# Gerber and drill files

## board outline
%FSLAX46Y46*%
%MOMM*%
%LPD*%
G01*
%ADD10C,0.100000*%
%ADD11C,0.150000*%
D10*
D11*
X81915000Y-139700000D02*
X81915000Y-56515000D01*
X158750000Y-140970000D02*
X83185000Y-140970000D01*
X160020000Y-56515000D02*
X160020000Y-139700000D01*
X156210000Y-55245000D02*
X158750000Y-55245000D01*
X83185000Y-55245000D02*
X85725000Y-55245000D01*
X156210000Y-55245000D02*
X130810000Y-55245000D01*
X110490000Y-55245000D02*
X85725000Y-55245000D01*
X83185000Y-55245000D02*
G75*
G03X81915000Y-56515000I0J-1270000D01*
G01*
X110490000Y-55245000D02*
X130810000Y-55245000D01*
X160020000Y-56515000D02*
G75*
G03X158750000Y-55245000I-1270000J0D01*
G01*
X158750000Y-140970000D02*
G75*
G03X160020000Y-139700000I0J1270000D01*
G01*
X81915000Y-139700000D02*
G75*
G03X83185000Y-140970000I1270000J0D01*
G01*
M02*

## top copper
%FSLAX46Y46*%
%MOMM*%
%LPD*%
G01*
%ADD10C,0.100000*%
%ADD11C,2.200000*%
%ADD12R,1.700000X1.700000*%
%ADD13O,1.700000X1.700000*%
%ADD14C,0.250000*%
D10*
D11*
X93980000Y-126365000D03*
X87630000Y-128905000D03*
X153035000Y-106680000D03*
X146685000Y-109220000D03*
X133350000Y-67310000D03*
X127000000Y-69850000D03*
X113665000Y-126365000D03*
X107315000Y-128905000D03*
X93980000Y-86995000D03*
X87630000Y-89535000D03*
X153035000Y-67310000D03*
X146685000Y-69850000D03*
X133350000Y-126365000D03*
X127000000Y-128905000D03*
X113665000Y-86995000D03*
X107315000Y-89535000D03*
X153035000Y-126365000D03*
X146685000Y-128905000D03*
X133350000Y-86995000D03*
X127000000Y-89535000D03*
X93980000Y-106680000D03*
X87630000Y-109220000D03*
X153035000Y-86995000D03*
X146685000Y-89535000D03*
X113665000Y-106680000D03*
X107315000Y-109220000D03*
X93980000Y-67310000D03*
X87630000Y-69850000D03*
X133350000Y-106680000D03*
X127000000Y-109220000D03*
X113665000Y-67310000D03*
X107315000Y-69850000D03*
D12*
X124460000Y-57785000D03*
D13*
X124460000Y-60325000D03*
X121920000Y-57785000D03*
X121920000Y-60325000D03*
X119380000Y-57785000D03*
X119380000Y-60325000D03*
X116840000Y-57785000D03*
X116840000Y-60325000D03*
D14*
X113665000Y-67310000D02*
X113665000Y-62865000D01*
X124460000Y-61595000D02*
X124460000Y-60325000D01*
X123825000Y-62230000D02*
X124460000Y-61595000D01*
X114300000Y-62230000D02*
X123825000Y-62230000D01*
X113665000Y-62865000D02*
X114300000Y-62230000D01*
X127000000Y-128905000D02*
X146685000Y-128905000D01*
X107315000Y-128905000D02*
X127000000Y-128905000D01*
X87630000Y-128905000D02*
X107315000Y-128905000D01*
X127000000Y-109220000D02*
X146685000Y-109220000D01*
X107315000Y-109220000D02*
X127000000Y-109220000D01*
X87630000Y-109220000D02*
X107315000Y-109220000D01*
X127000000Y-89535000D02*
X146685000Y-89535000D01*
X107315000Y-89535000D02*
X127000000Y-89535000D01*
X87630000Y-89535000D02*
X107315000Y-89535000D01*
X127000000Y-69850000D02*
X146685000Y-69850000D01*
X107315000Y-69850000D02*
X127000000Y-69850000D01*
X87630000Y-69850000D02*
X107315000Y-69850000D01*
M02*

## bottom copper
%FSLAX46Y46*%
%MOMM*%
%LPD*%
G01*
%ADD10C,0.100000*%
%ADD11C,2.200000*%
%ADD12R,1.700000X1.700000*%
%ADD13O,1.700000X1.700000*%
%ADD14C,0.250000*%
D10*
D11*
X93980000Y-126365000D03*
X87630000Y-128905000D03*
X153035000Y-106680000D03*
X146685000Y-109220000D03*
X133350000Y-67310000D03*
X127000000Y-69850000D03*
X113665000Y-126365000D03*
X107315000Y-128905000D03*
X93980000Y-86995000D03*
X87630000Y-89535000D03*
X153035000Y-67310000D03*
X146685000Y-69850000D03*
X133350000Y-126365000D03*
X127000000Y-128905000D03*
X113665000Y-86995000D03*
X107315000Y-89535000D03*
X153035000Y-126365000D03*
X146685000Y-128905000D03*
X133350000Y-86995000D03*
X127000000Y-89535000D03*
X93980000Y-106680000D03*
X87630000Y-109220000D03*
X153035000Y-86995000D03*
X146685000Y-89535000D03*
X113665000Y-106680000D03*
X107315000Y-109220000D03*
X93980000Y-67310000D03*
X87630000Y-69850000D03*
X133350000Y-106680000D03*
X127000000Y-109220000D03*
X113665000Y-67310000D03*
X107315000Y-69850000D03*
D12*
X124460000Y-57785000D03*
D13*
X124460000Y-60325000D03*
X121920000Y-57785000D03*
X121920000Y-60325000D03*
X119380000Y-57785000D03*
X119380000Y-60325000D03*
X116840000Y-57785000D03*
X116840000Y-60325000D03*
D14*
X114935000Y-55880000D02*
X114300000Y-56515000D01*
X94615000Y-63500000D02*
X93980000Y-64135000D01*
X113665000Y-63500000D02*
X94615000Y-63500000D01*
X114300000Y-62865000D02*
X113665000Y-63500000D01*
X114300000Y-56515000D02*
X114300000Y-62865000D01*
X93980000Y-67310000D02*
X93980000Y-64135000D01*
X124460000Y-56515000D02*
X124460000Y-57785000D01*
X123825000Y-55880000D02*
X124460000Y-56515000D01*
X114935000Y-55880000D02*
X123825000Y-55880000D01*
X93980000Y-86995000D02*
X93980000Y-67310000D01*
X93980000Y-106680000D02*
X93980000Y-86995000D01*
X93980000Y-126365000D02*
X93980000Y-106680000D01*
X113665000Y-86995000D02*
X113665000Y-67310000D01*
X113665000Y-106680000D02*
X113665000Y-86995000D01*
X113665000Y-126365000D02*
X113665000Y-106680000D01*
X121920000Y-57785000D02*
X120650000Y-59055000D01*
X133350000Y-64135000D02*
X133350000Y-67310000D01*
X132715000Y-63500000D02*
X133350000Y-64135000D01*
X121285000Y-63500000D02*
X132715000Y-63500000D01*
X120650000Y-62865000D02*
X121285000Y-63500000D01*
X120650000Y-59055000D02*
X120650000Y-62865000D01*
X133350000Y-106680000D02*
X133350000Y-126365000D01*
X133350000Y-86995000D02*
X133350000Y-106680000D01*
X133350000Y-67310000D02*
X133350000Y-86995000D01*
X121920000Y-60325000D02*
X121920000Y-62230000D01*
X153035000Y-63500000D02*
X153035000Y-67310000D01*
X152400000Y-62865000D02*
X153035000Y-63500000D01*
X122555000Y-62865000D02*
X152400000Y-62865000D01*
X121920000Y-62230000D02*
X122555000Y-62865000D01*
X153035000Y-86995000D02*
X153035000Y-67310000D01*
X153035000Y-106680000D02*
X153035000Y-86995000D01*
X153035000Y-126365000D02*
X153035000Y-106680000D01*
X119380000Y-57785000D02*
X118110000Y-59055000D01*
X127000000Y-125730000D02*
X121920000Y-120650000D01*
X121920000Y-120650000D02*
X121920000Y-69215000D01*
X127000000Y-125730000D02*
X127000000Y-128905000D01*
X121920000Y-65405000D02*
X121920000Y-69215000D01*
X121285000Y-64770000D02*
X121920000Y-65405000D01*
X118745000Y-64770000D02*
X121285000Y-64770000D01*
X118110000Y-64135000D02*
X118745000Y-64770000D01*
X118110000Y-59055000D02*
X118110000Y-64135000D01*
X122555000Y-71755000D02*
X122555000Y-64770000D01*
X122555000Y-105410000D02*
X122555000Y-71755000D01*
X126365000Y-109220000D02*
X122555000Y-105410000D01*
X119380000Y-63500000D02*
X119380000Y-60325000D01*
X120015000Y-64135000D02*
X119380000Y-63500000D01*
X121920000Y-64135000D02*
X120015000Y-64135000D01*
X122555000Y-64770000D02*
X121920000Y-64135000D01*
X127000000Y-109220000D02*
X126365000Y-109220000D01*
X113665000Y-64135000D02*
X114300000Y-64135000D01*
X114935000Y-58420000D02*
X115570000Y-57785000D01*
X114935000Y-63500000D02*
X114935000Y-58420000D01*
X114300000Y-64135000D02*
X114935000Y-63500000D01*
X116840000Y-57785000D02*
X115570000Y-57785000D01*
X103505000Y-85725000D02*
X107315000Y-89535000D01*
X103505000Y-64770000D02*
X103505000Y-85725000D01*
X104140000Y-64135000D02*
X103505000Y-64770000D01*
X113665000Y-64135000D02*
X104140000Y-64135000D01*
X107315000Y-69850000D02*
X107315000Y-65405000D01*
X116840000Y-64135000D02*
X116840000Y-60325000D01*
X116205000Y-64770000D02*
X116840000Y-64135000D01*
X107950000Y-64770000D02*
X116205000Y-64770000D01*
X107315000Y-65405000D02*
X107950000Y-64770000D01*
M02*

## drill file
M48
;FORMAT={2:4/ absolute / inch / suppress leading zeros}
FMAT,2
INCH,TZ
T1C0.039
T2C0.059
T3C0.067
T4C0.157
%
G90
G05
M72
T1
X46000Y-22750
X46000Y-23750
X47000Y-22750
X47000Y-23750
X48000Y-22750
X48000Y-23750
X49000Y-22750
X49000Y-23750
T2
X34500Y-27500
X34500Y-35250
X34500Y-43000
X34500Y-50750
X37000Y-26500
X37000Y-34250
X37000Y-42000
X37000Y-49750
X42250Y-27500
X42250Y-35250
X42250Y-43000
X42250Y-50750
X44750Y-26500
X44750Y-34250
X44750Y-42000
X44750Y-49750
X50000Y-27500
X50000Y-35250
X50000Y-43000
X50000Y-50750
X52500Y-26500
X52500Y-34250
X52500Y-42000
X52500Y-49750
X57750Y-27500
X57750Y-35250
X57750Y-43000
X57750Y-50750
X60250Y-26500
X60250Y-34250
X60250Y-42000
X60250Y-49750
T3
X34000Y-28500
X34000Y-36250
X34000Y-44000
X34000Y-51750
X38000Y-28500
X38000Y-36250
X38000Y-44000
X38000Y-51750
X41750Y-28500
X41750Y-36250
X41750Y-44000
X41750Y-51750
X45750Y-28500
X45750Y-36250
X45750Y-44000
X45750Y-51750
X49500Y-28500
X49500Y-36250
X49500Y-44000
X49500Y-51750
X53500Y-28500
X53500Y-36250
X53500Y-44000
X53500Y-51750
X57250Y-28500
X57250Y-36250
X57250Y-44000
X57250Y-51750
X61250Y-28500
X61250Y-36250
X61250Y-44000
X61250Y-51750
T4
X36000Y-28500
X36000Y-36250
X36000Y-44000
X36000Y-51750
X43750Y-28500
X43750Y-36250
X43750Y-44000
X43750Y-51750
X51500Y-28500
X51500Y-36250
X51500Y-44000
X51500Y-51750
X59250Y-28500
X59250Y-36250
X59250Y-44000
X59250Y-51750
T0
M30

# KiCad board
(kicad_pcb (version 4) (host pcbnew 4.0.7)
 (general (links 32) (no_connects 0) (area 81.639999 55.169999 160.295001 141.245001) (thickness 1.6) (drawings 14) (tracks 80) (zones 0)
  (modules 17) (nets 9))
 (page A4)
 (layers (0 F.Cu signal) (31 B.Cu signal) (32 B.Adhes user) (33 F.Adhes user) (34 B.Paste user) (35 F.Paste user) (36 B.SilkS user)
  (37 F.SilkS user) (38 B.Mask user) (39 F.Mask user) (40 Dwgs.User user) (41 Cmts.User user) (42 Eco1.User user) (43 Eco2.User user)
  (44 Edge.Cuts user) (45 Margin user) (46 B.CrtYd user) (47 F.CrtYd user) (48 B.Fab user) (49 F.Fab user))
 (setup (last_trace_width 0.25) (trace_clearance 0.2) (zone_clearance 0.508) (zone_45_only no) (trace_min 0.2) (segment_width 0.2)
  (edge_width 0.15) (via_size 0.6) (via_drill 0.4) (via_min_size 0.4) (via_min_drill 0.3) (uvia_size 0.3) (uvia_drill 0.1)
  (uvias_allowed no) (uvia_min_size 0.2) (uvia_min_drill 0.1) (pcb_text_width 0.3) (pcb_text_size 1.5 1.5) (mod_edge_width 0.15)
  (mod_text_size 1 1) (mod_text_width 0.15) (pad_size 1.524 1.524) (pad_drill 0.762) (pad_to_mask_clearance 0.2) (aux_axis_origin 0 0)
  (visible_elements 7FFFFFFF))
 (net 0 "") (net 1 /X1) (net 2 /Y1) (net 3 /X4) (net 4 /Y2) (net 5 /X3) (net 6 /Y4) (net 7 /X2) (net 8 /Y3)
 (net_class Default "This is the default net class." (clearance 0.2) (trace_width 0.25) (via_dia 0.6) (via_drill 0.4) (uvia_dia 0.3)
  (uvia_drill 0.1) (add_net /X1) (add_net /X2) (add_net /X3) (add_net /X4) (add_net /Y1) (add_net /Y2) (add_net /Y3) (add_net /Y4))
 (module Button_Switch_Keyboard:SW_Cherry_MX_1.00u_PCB (layer F.Cu) (at 93.98 126.365)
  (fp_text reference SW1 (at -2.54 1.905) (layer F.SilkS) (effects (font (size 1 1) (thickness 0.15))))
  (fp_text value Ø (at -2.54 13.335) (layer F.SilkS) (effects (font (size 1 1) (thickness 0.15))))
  (pad 1 thru_hole circle (at 0 0) (size 2.2 2.2) (drill 1.5) (layers *.Cu *.Mask) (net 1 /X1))
  (pad 2 thru_hole circle (at -6.35 2.54) (size 2.2 2.2) (drill 1.5) (layers *.Cu *.Mask) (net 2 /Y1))
  (pad "" np_thru_hole circle (at -2.54 5.08) (size 4 4) (drill 4) (layers *.Cu *.Mask))
  (pad "" np_thru_hole circle (at -7.62 5.08) (size 1.7 1.7) (drill 1.7) (layers *.Cu *.Mask))
  (pad "" np_thru_hole circle (at 2.54 5.08) (size 1.7 1.7) (drill 1.7) (layers *.Cu *.Mask)))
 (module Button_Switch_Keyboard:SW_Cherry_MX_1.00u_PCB (layer F.Cu) (at 153.035 106.68)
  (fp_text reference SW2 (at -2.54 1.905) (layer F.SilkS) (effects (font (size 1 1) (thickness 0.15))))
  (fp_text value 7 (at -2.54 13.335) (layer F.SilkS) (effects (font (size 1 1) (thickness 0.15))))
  (pad 1 thru_hole circle (at 0 0) (size 2.2 2.2) (drill 1.5) (layers *.Cu *.Mask) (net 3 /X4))
  (pad 2 thru_hole circle (at -6.35 2.54) (size 2.2 2.2) (drill 1.5) (layers *.Cu *.Mask) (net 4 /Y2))
  (pad "" np_thru_hole circle (at -2.54 5.08) (size 4 4) (drill 4) (layers *.Cu *.Mask))
  (pad "" np_thru_hole circle (at -7.62 5.08) (size 1.7 1.7) (drill 1.7) (layers *.Cu *.Mask))
  (pad "" np_thru_hole circle (at 2.54 5.08) (size 1.7 1.7) (drill 1.7) (layers *.Cu *.Mask)))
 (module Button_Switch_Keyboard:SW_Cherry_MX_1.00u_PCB (layer F.Cu) (at 133.35 67.31)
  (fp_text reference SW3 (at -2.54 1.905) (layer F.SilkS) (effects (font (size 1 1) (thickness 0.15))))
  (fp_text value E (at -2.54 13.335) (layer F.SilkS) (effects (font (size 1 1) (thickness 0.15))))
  (pad 1 thru_hole circle (at 0 0) (size 2.2 2.2) (drill 1.5) (layers *.Cu *.Mask) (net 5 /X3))
  (pad 2 thru_hole circle (at -6.35 2.54) (size 2.2 2.2) (drill 1.5) (layers *.Cu *.Mask) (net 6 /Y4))
  (pad "" np_thru_hole circle (at -2.54 5.08) (size 4 4) (drill 4) (layers *.Cu *.Mask))
  (pad "" np_thru_hole circle (at -7.62 5.08) (size 1.7 1.7) (drill 1.7) (layers *.Cu *.Mask))
  (pad "" np_thru_hole circle (at 2.54 5.08) (size 1.7 1.7) (drill 1.7) (layers *.Cu *.Mask)))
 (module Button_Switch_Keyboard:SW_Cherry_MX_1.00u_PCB (layer F.Cu) (at 113.665 126.365)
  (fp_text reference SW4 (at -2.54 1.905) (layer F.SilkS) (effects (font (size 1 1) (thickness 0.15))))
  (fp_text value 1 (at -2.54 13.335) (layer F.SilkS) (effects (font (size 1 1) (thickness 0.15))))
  (pad 1 thru_hole circle (at 0 0) (size 2.2 2.2) (drill 1.5) (layers *.Cu *.Mask) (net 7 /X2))
  (pad 2 thru_hole circle (at -6.35 2.54) (size 2.2 2.2) (drill 1.5) (layers *.Cu *.Mask) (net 2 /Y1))
  (pad "" np_thru_hole circle (at -2.54 5.08) (size 4 4) (drill 4) (layers *.Cu *.Mask))
  (pad "" np_thru_hole circle (at -7.62 5.08) (size 1.7 1.7) (drill 1.7) (layers *.Cu *.Mask))
  (pad "" np_thru_hole circle (at 2.54 5.08) (size 1.7 1.7) (drill 1.7) (layers *.Cu *.Mask)))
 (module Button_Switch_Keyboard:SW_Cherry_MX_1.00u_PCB (layer F.Cu) (at 93.98 86.995)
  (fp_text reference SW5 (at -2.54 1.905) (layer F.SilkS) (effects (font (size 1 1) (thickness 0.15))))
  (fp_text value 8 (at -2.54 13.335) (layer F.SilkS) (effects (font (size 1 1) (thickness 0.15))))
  (pad 1 thru_hole circle (at 0 0) (size 2.2 2.2) (drill 1.5) (layers *.Cu *.Mask) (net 1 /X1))
  (pad 2 thru_hole circle (at -6.35 2.54) (size 2.2 2.2) (drill 1.5) (layers *.Cu *.Mask) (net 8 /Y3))
  (pad "" np_thru_hole circle (at -2.54 5.08) (size 4 4) (drill 4) (layers *.Cu *.Mask))
  (pad "" np_thru_hole circle (at -7.62 5.08) (size 1.7 1.7) (drill 1.7) (layers *.Cu *.Mask))
  (pad "" np_thru_hole circle (at 2.54 5.08) (size 1.7 1.7) (drill 1.7) (layers *.Cu *.Mask)))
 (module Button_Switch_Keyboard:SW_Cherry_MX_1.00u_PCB (layer F.Cu) (at 153.035 67.31)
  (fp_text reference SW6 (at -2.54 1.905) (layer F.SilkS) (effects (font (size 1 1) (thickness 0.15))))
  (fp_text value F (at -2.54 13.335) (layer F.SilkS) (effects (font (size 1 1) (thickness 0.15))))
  (pad 1 thru_hole circle (at 0 0) (size 2.2 2.2) (drill 1.5) (layers *.Cu *.Mask) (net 3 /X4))
  (pad 2 thru_hole circle (at -6.35 2.54) (size 2.2 2.2) (drill 1.5) (layers *.Cu *.Mask) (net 6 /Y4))
  (pad "" np_thru_hole circle (at -2.54 5.08) (size 4 4) (drill 4) (layers *.Cu *.Mask))
  (pad "" np_thru_hole circle (at -7.62 5.08) (size 1.7 1.7) (drill 1.7) (layers *.Cu *.Mask))
  (pad "" np_thru_hole circle (at 2.54 5.08) (size 1.7 1.7) (drill 1.7) (layers *.Cu *.Mask)))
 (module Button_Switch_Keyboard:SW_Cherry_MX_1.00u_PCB (layer F.Cu) (at 133.35 126.365)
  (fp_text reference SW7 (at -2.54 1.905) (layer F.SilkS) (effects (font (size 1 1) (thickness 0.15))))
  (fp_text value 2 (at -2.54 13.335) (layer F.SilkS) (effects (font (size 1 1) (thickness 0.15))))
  (pad 1 thru_hole circle (at 0 0) (size 2.2 2.2) (drill 1.5) (layers *.Cu *.Mask) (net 5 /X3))
  (pad 2 thru_hole circle (at -6.35 2.54) (size 2.2 2.2) (drill 1.5) (layers *.Cu *.Mask) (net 2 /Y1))
  (pad "" np_thru_hole circle (at -2.54 5.08) (size 4 4) (drill 4) (layers *.Cu *.Mask))
  (pad "" np_thru_hole circle (at -7.62 5.08) (size 1.7 1.7) (drill 1.7) (layers *.Cu *.Mask))
  (pad "" np_thru_hole circle (at 2.54 5.08) (size 1.7 1.7) (drill 1.7) (layers *.Cu *.Mask)))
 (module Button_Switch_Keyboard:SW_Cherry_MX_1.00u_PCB (layer F.Cu) (at 113.665 86.995)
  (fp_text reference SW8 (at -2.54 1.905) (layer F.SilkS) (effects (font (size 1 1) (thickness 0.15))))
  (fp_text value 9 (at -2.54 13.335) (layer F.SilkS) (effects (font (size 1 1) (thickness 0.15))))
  (pad 1 thru_hole circle (at 0 0) (size 2.2 2.2) (drill 1.5) (layers *.Cu *.Mask) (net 7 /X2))
  (pad 2 thru_hole circle (at -6.35 2.54) (size 2.2 2.2) (drill 1.5) (layers *.Cu *.Mask) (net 8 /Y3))
  (pad "" np_thru_hole circle (at -2.54 5.08) (size 4 4) (drill 4) (layers *.Cu *.Mask))
  (pad "" np_thru_hole circle (at -7.62 5.08) (size 1.7 1.7) (drill 1.7) (layers *.Cu *.Mask))
  (pad "" np_thru_hole circle (at 2.54 5.08) (size 1.7 1.7) (drill 1.7) (layers *.Cu *.Mask)))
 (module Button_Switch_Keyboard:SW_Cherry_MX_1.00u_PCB (layer F.Cu) (at 153.035 126.365)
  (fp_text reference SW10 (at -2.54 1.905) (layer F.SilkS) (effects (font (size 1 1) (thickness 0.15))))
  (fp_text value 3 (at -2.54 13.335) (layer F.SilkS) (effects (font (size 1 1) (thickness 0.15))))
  (pad 1 thru_hole circle (at 0 0) (size 2.2 2.2) (drill 1.5) (layers *.Cu *.Mask) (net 3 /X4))
  (pad 2 thru_hole circle (at -6.35 2.54) (size 2.2 2.2) (drill 1.5) (layers *.Cu *.Mask) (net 2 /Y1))
  (pad "" np_thru_hole circle (at -2.54 5.08) (size 4 4) (drill 4) (layers *.Cu *.Mask))
  (pad "" np_thru_hole circle (at -7.62 5.08) (size 1.7 1.7) (drill 1.7) (layers *.Cu *.Mask))
  (pad "" np_thru_hole circle (at 2.54 5.08) (size 1.7 1.7) (drill 1.7) (layers *.Cu *.Mask)))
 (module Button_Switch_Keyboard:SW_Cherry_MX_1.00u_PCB (layer F.Cu) (at 133.35 86.995)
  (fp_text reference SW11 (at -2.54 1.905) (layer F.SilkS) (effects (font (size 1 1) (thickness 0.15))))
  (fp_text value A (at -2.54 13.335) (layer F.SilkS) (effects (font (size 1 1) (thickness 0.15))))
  (pad 1 thru_hole circle (at 0 0) (size 2.2 2.2) (drill 1.5) (layers *.Cu *.Mask) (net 5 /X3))
  (pad 2 thru_hole circle (at -6.35 2.54) (size 2.2 2.2) (drill 1.5) (layers *.Cu *.Mask) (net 8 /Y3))
  (pad "" np_thru_hole circle (at -2.54 5.08) (size 4 4) (drill 4) (layers *.Cu *.Mask))
  (pad "" np_thru_hole circle (at -7.62 5.08) (size 1.7 1.7) (drill 1.7) (layers *.Cu *.Mask))
  (pad "" np_thru_hole circle (at 2.54 5.08) (size 1.7 1.7) (drill 1.7) (layers *.Cu *.Mask)))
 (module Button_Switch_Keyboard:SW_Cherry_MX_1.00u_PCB (layer F.Cu) (at 93.98 106.68)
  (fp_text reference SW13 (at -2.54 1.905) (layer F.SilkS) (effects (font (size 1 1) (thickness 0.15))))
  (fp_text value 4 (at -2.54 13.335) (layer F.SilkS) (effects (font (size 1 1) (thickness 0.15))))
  (pad 1 thru_hole circle (at 0 0) (size 2.2 2.2) (drill 1.5) (layers *.Cu *.Mask) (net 1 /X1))
  (pad 2 thru_hole circle (at -6.35 2.54) (size 2.2 2.2) (drill 1.5) (layers *.Cu *.Mask) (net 4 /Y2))
  (pad "" np_thru_hole circle (at -2.54 5.08) (size 4 4) (drill 4) (layers *.Cu *.Mask))
  (pad "" np_thru_hole circle (at -7.62 5.08) (size 1.7 1.7) (drill 1.7) (layers *.Cu *.Mask))
  (pad "" np_thru_hole circle (at 2.54 5.08) (size 1.7 1.7) (drill 1.7) (layers *.Cu *.Mask)))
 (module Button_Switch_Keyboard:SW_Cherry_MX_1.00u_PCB (layer F.Cu) (at 153.035 86.995)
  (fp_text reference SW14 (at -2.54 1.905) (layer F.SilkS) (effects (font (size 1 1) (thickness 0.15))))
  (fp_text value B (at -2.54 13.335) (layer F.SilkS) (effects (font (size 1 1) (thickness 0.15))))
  (pad 1 thru_hole circle (at 0 0) (size 2.2 2.2) (drill 1.5) (layers *.Cu *.Mask) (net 3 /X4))
  (pad 2 thru_hole circle (at -6.35 2.54) (size 2.2 2.2) (drill 1.5) (layers *.Cu *.Mask) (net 8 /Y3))
  (pad "" np_thru_hole circle (at -2.54 5.08) (size 4 4) (drill 4) (layers *.Cu *.Mask))
  (pad "" np_thru_hole circle (at -7.62 5.08) (size 1.7 1.7) (drill 1.7) (layers *.Cu *.Mask))
  (pad "" np_thru_hole circle (at 2.54 5.08) (size 1.7 1.7) (drill 1.7) (layers *.Cu *.Mask)))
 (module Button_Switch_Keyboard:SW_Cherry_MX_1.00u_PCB (layer F.Cu) (at 113.665 106.68)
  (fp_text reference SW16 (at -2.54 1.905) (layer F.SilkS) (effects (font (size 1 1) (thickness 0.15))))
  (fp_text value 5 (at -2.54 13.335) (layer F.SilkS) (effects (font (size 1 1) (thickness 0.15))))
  (pad 1 thru_hole circle (at 0 0) (size 2.2 2.2) (drill 1.5) (layers *.Cu *.Mask) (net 7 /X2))
  (pad 2 thru_hole circle (at -6.35 2.54) (size 2.2 2.2) (drill 1.5) (layers *.Cu *.Mask) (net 4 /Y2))
  (pad "" np_thru_hole circle (at -2.54 5.08) (size 4 4) (drill 4) (layers *.Cu *.Mask))
  (pad "" np_thru_hole circle (at -7.62 5.08) (size 1.7 1.7) (drill 1.7) (layers *.Cu *.Mask))
  (pad "" np_thru_hole circle (at 2.54 5.08) (size 1.7 1.7) (drill 1.7) (layers *.Cu *.Mask)))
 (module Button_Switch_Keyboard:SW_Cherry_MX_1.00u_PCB (layer F.Cu) (at 93.98 67.31)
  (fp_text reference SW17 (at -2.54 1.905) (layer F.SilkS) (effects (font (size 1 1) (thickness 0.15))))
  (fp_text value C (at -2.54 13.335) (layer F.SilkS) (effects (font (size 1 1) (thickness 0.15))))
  (pad 1 thru_hole circle (at 0 0) (size 2.2 2.2) (drill 1.5) (layers *.Cu *.Mask) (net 1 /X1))
  (pad 2 thru_hole circle (at -6.35 2.54) (size 2.2 2.2) (drill 1.5) (layers *.Cu *.Mask) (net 6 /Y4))
  (pad "" np_thru_hole circle (at -2.54 5.08) (size 4 4) (drill 4) (layers *.Cu *.Mask))
  (pad "" np_thru_hole circle (at -7.62 5.08) (size 1.7 1.7) (drill 1.7) (layers *.Cu *.Mask))
  (pad "" np_thru_hole circle (at 2.54 5.08) (size 1.7 1.7) (drill 1.7) (layers *.Cu *.Mask)))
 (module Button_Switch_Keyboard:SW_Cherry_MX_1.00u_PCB (layer F.Cu) (at 133.35 106.68)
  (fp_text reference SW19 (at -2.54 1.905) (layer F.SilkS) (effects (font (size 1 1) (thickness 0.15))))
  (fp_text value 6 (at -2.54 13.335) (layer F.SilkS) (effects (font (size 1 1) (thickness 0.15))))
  (pad 1 thru_hole circle (at 0 0) (size 2.2 2.2) (drill 1.5) (layers *.Cu *.Mask) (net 5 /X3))
  (pad 2 thru_hole circle (at -6.35 2.54) (size 2.2 2.2) (drill 1.5) (layers *.Cu *.Mask) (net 4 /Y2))
  (pad "" np_thru_hole circle (at -2.54 5.08) (size 4 4) (drill 4) (layers *.Cu *.Mask))
  (pad "" np_thru_hole circle (at -7.62 5.08) (size 1.7 1.7) (drill 1.7) (layers *.Cu *.Mask))
  (pad "" np_thru_hole circle (at 2.54 5.08) (size 1.7 1.7) (drill 1.7) (layers *.Cu *.Mask)))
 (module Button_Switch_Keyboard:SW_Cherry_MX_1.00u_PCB (layer F.Cu) (at 113.665 67.31)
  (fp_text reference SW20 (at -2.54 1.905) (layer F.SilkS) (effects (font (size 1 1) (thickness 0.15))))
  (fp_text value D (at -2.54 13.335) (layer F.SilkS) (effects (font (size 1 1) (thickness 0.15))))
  (pad 1 thru_hole circle (at 0 0) (size 2.2 2.2) (drill 1.5) (layers *.Cu *.Mask) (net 7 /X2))
  (pad 2 thru_hole circle (at -6.35 2.54) (size 2.2 2.2) (drill 1.5) (layers *.Cu *.Mask) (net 6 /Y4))
  (pad "" np_thru_hole circle (at -2.54 5.08) (size 4 4) (drill 4) (layers *.Cu *.Mask))
  (pad "" np_thru_hole circle (at -7.62 5.08) (size 1.7 1.7) (drill 1.7) (layers *.Cu *.Mask))
  (pad "" np_thru_hole circle (at 2.54 5.08) (size 1.7 1.7) (drill 1.7) (layers *.Cu *.Mask)))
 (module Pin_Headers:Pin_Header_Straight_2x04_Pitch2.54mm (layer F.Cu) (at 124.46 57.785 270)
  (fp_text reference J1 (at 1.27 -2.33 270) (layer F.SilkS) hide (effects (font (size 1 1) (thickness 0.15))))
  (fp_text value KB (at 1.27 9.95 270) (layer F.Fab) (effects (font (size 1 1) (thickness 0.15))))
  (pad 1 thru_hole rect (at 0 0 270) (size 1.7 1.7) (drill 1) (layers *.Cu *.Mask) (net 1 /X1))
  (pad 2 thru_hole oval (at 2.54 0 270) (size 1.7 1.7) (drill 1) (layers *.Cu *.Mask) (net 7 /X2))
  (pad 3 thru_hole oval (at 0 2.54 270) (size 1.7 1.7) (drill 1) (layers *.Cu *.Mask) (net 5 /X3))
  (pad 4 thru_hole oval (at 2.54 2.54 270) (size 1.7 1.7) (drill 1) (layers *.Cu *.Mask) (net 3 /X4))
  (pad 5 thru_hole oval (at 0 5.08 270) (size 1.7 1.7) (drill 1) (layers *.Cu *.Mask) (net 2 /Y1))
  (pad 6 thru_hole oval (at 2.54 5.08 270) (size 1.7 1.7) (drill 1) (layers *.Cu *.Mask) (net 4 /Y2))
  (pad 7 thru_hole oval (at 0 7.62 270) (size 1.7 1.7) (drill 1) (layers *.Cu *.Mask) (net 8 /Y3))
  (pad 8 thru_hole oval (at 2.54 7.62 270) (size 1.7 1.7) (drill 1) (layers *.Cu *.Mask) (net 6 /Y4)))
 (gr_line (start 81.915 139.7) (end 81.915 56.515) (angle 90) (layer Edge.Cuts) (width 0.15))
 (gr_line (start 158.75 140.97) (end 83.185 140.97) (angle 90) (layer Edge.Cuts) (width 0.15))
 (gr_line (start 160.02 56.515) (end 160.02 139.7) (angle 90) (layer Edge.Cuts) (width 0.15))
 (gr_line (start 156.21 55.245) (end 158.75 55.245) (angle 90) (layer Edge.Cuts) (width 0.15))
 (gr_line (start 83.185 55.245) (end 85.725 55.245) (angle 90) (layer Edge.Cuts) (width 0.15))
 (gr_line (start 156.21 55.245) (end 130.81 55.245) (angle 90) (layer Edge.Cuts) (width 0.15))
 (gr_line (start 110.49 55.245) (end 85.725 55.245) (angle 90) (layer Edge.Cuts) (width 0.15))
 (gr_arc (start 83.185 56.515) (end 81.915 56.515) (angle 90) (layer Edge.Cuts) (width 0.15))
 (gr_line (start 110.49 55.245) (end 130.81 55.245) (angle 90) (layer Edge.Cuts) (width 0.15))
 (gr_arc (start 158.75 56.515) (end 158.75 55.245) (angle 90) (layer Edge.Cuts) (width 0.15))
 (gr_arc (start 158.75 139.7) (end 160.02 139.7) (angle 90) (layer Edge.Cuts) (width 0.15))
 (gr_arc (start 83.185 139.7) (end 83.185 140.97) (angle 90) (layer Edge.Cuts) (width 0.15))
 (segment (start 114.935 55.88) (end 114.3 56.515) (width 0.25) (layer B.Cu) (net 1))
 (segment (start 94.615 63.5) (end 93.98 64.135) (width 0.25) (layer B.Cu) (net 1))
 (segment (start 113.665 63.5) (end 94.615 63.5) (width 0.25) (layer B.Cu) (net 1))
 (segment (start 114.3 62.865) (end 113.665 63.5) (width 0.25) (layer B.Cu) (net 1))
 (segment (start 114.3 56.515) (end 114.3 62.865) (width 0.25) (layer B.Cu) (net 1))
 (segment (start 93.98 67.31) (end 93.98 64.135) (width 0.25) (layer B.Cu) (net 1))
 (segment (start 124.46 56.515) (end 124.46 57.785) (width 0.25) (layer B.Cu) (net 1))
 (segment (start 123.825 55.88) (end 124.46 56.515) (width 0.25) (layer B.Cu) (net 1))
 (segment (start 114.935 55.88) (end 123.825 55.88) (width 0.25) (layer B.Cu) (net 1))
 (segment (start 93.98 86.995) (end 93.98 67.31) (width 0.25) (layer B.Cu) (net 1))
 (segment (start 93.98 106.68) (end 93.98 86.995) (width 0.25) (layer B.Cu) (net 1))
 (segment (start 93.98 126.365) (end 93.98 106.68) (width 0.25) (layer B.Cu) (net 1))
 (segment (start 113.665 67.31) (end 113.665 62.865) (width 0.25) (layer F.Cu) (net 7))
 (segment (start 124.46 61.595) (end 124.46 60.325) (width 0.25) (layer F.Cu) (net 7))
 (segment (start 123.825 62.23) (end 124.46 61.595) (width 0.25) (layer F.Cu) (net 7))
 (segment (start 114.3 62.23) (end 123.825 62.23) (width 0.25) (layer F.Cu) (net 7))
 (segment (start 113.665 62.865) (end 114.3 62.23) (width 0.25) (layer F.Cu) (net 7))
 (segment (start 113.665 86.995) (end 113.665 67.31) (width 0.25) (layer B.Cu) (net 7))
 (segment (start 113.665 106.68) (end 113.665 86.995) (width 0.25) (layer B.Cu) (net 7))
 (segment (start 113.665 126.365) (end 113.665 106.68) (width 0.25) (layer B.Cu) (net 7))
 (segment (start 121.92 57.785) (end 120.65 59.055) (width 0.25) (layer B.Cu) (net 5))
 (segment (start 133.35 64.135) (end 133.35 67.31) (width 0.25) (layer B.Cu) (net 5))
 (segment (start 132.715 63.5) (end 133.35 64.135) (width 0.25) (layer B.Cu) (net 5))
 (segment (start 121.285 63.5) (end 132.715 63.5) (width 0.25) (layer B.Cu) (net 5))
 (segment (start 120.65 62.865) (end 121.285 63.5) (width 0.25) (layer B.Cu) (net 5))
 (segment (start 120.65 59.055) (end 120.65 62.865) (width 0.25) (layer B.Cu) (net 5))
 (segment (start 133.35 106.68) (end 133.35 126.365) (width 0.25) (layer B.Cu) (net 5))
 (segment (start 133.35 86.995) (end 133.35 106.68) (width 0.25) (layer B.Cu) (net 5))
 (segment (start 133.35 67.31) (end 133.35 86.995) (width 0.25) (layer B.Cu) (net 5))
 (segment (start 121.92 60.325) (end 121.92 62.23) (width 0.25) (layer B.Cu) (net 3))
 (segment (start 153.035 63.5) (end 153.035 67.31) (width 0.25) (layer B.Cu) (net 3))
 (segment (start 152.4 62.865) (end 153.035 63.5) (width 0.25) (layer B.Cu) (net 3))
 (segment (start 122.555 62.865) (end 152.4 62.865) (width 0.25) (layer B.Cu) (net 3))
 (segment (start 121.92 62.23) (end 122.555 62.865) (width 0.25) (layer B.Cu) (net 3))
 (segment (start 153.035 86.995) (end 153.035 67.31) (width 0.25) (layer B.Cu) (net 3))
 (segment (start 153.035 106.68) (end 153.035 86.995) (width 0.25) (layer B.Cu) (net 3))
 (segment (start 153.035 126.365) (end 153.035 106.68) (width 0.25) (layer B.Cu) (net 3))
 (segment (start 119.38 57.785) (end 118.11 59.055) (width 0.25) (layer B.Cu) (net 2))
 (segment (start 127 125.73) (end 121.92 120.65) (width 0.25) (layer B.Cu) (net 2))
 (segment (start 121.92 120.65) (end 121.92 69.215) (width 0.25) (layer B.Cu) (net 2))
 (segment (start 127 125.73) (end 127 128.905) (width 0.25) (layer B.Cu) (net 2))
 (segment (start 121.92 65.405) (end 121.92 69.215) (width 0.25) (layer B.Cu) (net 2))
 (segment (start 121.285 64.77) (end 121.92 65.405) (width 0.25) (layer B.Cu) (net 2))
 (segment (start 118.745 64.77) (end 121.285 64.77) (width 0.25) (layer B.Cu) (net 2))
 (segment (start 118.11 64.135) (end 118.745 64.77) (width 0.25) (layer B.Cu) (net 2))
 (segment (start 118.11 59.055) (end 118.11 64.135) (width 0.25) (layer B.Cu) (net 2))
 (segment (start 127 128.905) (end 146.685 128.905) (width 0.25) (layer F.Cu) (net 2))
 (segment (start 107.315 128.905) (end 127 128.905) (width 0.25) (layer F.Cu) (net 2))
 (segment (start 87.63 128.905) (end 107.315 128.905) (width 0.25) (layer F.Cu) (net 2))
 (segment (start 122.555 71.755) (end 122.555 64.77) (width 0.25) (layer B.Cu) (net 4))
 (segment (start 122.555 105.41) (end 122.555 71.755) (width 0.25) (layer B.Cu) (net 4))
 (segment (start 126.365 109.22) (end 122.555 105.41) (width 0.25) (layer B.Cu) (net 4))
 (segment (start 119.38 63.5) (end 119.38 60.325) (width 0.25) (layer B.Cu) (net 4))
 (segment (start 120.015 64.135) (end 119.38 63.5) (width 0.25) (layer B.Cu) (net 4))
 (segment (start 121.92 64.135) (end 120.015 64.135) (width 0.25) (layer B.Cu) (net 4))
 (segment (start 122.555 64.77) (end 121.92 64.135) (width 0.25) (layer B.Cu) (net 4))
 (segment (start 127 109.22) (end 126.365 109.22) (width 0.25) (layer B.Cu) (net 4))
 (segment (start 127 109.22) (end 146.685 109.22) (width 0.25) (layer F.Cu) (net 4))
 (segment (start 107.315 109.22) (end 127 109.22) (width 0.25) (layer F.Cu) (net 4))
 (segment (start 87.63 109.22) (end 107.315 109.22) (width 0.25) (layer F.Cu) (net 4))
 (segment (start 113.665 64.135) (end 114.3 64.135) (width 0.25) (layer B.Cu) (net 8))
 (segment (start 114.935 58.42) (end 115.57 57.785) (width 0.25) (layer B.Cu) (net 8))
 (segment (start 114.935 63.5) (end 114.935 58.42) (width 0.25) (layer B.Cu) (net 8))
 (segment (start 114.3 64.135) (end 114.935 63.5) (width 0.25) (layer B.Cu) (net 8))
 (segment (start 116.84 57.785) (end 115.57 57.785) (width 0.25) (layer B.Cu) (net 8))
 (segment (start 103.505 85.725) (end 107.315 89.535) (width 0.25) (layer B.Cu) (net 8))
 (segment (start 103.505 64.77) (end 103.505 85.725) (width 0.25) (layer B.Cu) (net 8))
 (segment (start 104.14 64.135) (end 103.505 64.77) (width 0.25) (layer B.Cu) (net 8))
 (segment (start 113.665 64.135) (end 104.14 64.135) (width 0.25) (layer B.Cu) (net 8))
 (segment (start 127 89.535) (end 146.685 89.535) (width 0.25) (layer F.Cu) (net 8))
 (segment (start 107.315 89.535) (end 127 89.535) (width 0.25) (layer F.Cu) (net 8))
 (segment (start 87.63 89.535) (end 107.315 89.535) (width 0.25) (layer F.Cu) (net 8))
 (segment (start 107.315 69.85) (end 107.315 65.405) (width 0.25) (layer B.Cu) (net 6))
 (segment (start 116.84 64.135) (end 116.84 60.325) (width 0.25) (layer B.Cu) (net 6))
 (segment (start 116.205 64.77) (end 116.84 64.135) (width 0.25) (layer B.Cu) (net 6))
 (segment (start 107.95 64.77) (end 116.205 64.77) (width 0.25) (layer B.Cu) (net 6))
 (segment (start 107.315 65.405) (end 107.95 64.77) (width 0.25) (layer B.Cu) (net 6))
 (segment (start 127 69.85) (end 146.685 69.85) (width 0.25) (layer F.Cu) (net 6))
 (segment (start 107.315 69.85) (end 127 69.85) (width 0.25) (layer F.Cu) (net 6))
 (segment (start 87.63 69.85) (end 107.315 69.85) (width 0.25) (layer F.Cu) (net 6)))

